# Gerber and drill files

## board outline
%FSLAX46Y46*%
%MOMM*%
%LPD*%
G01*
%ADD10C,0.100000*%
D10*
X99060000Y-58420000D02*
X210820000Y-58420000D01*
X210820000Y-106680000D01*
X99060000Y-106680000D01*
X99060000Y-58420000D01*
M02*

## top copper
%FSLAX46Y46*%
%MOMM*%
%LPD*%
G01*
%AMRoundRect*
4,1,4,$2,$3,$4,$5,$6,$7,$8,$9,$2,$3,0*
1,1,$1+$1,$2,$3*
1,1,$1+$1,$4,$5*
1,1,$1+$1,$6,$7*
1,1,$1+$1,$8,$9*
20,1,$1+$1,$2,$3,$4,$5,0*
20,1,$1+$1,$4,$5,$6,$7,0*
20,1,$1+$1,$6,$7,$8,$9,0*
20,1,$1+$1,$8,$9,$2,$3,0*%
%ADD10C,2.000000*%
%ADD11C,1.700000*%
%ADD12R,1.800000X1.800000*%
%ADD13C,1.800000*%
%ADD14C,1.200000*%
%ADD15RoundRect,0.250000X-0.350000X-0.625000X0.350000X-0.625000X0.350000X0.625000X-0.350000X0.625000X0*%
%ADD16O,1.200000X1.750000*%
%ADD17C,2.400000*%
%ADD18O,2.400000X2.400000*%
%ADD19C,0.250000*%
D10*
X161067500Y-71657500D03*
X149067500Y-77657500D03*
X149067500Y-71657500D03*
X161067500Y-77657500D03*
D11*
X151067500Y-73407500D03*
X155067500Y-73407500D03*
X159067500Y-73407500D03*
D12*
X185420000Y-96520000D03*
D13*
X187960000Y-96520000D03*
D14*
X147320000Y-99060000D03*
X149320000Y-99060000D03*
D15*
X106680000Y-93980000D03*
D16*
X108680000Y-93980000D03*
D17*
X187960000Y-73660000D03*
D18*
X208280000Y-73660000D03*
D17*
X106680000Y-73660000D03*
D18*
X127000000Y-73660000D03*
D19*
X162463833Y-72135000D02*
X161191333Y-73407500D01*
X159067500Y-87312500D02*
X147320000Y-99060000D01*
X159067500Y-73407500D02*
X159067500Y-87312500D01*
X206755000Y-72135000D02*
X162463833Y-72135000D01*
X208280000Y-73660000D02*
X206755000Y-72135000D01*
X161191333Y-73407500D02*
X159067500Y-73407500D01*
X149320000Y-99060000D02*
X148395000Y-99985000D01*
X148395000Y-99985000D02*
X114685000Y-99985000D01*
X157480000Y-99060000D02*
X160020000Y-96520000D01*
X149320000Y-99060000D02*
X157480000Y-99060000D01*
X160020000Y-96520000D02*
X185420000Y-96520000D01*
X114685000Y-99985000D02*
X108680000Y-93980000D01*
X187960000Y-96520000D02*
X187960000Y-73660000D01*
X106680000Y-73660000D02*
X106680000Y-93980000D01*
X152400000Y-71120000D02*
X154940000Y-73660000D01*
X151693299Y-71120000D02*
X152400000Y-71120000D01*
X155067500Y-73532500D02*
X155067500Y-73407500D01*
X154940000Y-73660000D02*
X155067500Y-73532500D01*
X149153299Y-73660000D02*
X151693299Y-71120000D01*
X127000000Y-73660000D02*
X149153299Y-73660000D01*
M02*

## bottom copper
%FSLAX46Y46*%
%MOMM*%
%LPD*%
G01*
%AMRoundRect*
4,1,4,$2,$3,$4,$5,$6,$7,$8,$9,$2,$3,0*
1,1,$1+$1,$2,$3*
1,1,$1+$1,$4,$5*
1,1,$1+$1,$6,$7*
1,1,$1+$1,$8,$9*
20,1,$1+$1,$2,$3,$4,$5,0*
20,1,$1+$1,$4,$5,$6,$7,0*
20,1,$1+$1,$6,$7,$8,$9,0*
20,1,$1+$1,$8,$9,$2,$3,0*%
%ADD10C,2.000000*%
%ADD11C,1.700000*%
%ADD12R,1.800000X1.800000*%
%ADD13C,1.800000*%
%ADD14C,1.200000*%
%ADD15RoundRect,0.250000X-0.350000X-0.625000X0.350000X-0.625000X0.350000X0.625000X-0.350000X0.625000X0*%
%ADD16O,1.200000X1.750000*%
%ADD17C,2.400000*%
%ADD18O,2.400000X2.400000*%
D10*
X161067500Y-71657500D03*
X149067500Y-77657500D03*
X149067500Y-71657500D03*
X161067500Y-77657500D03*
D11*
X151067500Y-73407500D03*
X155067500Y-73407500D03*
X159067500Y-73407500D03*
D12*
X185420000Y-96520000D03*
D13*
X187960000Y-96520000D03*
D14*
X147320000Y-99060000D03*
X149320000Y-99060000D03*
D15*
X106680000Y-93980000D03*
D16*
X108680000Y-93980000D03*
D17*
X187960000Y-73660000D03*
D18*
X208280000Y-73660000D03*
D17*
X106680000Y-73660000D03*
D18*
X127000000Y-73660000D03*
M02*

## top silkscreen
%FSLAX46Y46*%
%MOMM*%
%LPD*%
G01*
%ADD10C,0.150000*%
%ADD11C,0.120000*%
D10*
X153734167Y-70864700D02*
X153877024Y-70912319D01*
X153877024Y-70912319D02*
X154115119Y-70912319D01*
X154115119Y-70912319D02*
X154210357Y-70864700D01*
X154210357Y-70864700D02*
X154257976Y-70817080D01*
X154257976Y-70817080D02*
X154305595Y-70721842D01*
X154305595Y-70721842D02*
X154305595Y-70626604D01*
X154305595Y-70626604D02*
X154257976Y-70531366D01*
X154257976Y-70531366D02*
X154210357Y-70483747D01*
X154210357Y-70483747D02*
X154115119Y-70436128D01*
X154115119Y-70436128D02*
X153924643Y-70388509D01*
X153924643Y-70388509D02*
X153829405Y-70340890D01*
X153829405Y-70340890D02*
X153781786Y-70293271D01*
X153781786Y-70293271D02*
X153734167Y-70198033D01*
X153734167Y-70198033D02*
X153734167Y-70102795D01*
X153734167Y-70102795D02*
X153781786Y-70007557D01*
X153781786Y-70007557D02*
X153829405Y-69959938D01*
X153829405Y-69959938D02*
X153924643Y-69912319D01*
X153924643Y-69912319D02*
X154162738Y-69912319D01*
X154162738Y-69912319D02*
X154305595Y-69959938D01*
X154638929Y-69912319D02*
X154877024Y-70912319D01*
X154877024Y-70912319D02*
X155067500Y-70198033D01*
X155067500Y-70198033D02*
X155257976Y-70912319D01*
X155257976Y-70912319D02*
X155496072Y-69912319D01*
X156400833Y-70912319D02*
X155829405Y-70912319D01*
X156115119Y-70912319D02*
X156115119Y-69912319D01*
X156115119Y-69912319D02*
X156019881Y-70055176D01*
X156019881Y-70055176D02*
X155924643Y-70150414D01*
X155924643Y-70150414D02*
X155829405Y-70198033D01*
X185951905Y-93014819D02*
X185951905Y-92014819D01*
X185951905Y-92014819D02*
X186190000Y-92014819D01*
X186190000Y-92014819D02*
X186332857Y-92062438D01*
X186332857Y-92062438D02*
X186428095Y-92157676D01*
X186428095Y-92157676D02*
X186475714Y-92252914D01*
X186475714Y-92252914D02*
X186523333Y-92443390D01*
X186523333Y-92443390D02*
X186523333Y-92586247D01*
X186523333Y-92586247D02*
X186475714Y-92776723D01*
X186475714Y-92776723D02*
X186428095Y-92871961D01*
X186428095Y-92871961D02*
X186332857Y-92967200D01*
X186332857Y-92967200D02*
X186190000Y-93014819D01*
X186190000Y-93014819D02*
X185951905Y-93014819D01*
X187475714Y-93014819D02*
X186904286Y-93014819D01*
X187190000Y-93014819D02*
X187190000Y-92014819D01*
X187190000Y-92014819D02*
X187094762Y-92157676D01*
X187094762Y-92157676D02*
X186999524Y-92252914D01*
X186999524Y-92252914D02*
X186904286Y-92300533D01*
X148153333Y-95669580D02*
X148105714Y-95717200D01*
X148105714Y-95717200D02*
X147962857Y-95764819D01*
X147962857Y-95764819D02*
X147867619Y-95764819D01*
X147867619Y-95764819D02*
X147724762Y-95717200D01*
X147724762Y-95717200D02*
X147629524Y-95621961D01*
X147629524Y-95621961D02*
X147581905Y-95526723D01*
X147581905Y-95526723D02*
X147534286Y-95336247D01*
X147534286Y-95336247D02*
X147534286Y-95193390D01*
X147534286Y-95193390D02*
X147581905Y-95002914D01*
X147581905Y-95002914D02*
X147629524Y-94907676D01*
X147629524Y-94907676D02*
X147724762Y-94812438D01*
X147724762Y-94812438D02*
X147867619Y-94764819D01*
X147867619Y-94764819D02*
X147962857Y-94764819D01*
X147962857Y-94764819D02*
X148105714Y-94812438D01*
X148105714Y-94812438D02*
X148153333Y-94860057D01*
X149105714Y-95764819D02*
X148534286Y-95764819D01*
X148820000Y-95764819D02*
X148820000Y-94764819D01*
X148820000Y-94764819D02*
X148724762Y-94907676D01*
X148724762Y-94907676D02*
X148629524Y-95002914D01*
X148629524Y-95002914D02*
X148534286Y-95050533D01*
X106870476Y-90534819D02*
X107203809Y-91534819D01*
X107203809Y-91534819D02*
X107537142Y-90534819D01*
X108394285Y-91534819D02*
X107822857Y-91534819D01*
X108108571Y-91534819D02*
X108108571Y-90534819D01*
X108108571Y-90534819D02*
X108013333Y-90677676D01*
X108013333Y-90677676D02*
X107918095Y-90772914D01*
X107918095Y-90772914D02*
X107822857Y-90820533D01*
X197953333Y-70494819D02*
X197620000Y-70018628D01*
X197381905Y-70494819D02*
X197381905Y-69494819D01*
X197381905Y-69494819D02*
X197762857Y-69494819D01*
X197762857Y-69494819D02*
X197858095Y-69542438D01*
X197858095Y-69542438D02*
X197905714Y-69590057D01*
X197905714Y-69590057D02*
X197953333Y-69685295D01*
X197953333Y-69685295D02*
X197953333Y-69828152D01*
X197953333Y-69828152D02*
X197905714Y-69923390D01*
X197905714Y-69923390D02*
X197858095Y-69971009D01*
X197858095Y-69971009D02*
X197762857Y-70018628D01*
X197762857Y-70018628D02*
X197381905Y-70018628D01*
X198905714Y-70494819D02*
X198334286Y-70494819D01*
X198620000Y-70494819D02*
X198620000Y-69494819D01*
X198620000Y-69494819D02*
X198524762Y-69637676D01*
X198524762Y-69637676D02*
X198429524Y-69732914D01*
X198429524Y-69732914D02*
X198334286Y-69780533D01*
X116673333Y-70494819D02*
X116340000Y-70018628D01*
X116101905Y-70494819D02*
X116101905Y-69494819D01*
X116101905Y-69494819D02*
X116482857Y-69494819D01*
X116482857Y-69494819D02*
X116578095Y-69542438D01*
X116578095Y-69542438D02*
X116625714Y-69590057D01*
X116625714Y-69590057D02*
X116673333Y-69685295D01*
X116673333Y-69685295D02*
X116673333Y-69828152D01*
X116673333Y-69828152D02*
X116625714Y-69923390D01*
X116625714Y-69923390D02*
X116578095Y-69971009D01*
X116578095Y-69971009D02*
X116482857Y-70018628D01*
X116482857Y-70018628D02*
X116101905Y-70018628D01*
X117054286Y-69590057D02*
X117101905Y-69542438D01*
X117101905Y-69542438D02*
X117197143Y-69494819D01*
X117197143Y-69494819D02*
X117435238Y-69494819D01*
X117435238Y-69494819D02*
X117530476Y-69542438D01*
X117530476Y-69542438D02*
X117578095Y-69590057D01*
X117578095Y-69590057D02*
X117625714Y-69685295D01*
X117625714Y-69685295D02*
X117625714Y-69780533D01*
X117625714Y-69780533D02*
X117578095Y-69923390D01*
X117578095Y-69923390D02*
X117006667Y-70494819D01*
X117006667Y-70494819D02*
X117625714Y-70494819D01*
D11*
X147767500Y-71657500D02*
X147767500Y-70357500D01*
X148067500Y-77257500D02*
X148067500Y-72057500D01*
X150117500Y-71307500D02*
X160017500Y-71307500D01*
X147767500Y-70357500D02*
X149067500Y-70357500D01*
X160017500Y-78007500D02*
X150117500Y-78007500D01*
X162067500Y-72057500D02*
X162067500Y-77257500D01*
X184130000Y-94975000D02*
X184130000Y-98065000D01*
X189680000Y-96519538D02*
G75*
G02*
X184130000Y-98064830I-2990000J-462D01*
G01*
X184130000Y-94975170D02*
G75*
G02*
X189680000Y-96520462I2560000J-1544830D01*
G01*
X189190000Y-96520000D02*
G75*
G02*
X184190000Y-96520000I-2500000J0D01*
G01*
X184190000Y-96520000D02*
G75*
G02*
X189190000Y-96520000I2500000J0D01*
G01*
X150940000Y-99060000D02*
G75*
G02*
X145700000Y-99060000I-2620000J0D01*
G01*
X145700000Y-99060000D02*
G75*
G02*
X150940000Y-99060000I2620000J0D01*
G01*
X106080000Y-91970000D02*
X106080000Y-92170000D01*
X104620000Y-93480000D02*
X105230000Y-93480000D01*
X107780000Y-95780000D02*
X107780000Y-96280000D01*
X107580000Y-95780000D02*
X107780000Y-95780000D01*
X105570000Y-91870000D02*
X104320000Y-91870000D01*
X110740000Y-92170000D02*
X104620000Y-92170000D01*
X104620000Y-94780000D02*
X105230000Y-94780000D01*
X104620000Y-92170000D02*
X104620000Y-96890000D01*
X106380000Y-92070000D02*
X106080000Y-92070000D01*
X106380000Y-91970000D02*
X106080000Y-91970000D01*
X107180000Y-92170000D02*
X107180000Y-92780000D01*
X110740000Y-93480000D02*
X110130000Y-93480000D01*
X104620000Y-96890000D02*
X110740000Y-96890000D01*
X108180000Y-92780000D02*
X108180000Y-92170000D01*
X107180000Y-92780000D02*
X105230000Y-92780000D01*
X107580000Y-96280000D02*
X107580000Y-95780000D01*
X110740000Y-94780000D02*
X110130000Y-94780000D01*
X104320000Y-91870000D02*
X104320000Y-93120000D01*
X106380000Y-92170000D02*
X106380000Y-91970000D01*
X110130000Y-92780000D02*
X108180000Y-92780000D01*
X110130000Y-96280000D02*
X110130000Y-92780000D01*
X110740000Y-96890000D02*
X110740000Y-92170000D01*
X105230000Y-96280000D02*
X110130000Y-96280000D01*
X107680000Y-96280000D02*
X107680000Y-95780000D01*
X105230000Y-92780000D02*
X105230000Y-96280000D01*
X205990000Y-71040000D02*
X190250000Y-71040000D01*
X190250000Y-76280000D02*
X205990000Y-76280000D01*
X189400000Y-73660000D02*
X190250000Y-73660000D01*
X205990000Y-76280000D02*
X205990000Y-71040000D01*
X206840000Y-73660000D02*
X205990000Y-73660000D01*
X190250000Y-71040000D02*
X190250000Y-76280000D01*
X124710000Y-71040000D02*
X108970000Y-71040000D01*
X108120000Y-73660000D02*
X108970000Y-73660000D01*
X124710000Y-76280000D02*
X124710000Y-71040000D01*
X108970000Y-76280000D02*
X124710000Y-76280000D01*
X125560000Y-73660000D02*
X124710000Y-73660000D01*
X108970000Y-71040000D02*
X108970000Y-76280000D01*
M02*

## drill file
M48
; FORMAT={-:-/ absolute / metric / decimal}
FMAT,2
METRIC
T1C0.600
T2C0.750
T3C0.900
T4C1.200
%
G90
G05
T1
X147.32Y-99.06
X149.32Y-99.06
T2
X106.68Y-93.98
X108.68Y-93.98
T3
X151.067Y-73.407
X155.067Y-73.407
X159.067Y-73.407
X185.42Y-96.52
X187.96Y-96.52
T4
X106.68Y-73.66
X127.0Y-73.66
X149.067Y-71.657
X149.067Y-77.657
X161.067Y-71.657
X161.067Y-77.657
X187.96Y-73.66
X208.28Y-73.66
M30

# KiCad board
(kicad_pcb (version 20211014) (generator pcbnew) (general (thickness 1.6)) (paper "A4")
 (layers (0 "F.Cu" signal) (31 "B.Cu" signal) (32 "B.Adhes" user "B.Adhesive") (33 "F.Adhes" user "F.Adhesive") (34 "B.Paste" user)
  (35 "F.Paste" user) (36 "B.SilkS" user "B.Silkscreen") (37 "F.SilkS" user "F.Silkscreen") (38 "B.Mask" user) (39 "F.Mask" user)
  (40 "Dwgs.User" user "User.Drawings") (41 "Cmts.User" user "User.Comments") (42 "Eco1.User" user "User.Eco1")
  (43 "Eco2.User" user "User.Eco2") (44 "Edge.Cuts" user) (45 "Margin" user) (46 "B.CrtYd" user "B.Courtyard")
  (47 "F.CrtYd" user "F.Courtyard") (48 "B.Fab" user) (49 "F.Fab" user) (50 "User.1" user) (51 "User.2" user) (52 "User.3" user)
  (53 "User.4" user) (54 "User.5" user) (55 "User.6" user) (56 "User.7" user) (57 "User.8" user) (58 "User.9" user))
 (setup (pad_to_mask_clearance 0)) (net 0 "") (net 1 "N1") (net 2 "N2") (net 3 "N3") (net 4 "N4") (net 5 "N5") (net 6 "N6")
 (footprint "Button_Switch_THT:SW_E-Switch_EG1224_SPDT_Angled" (layer "F.Cu") (at 151.0675 73.4075)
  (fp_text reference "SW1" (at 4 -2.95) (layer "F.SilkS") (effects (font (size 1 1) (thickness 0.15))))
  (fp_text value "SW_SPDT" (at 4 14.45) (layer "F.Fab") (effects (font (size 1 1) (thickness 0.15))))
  (fp_line (start -3.3 -1.75) (end -3.3 -3.05) (layer "F.SilkS") (width 0.12))
  (fp_line (start -3 3.85) (end -3 -1.35) (layer "F.SilkS") (width 0.12))
  (fp_line (start -0.95 -2.1) (end 8.95 -2.1) (layer "F.SilkS") (width 0.12))
  (fp_line (start -3.3 -3.05) (end -2 -3.05) (layer "F.SilkS") (width 0.12))
  (fp_line (start 8.95 4.6) (end -0.95 4.6) (layer "F.SilkS") (width 0.12))
  (fp_line (start 11 -1.35) (end 11 3.85) (layer "F.SilkS") (width 0.12))
  (pad "" thru_hole circle (at 10 -1.75) (size 2 2) (drill 1.2) (layers *.Cu *.Mask))
  (pad "" thru_hole circle (at -2 4.25) (size 2 2) (drill 1.2) (layers *.Cu *.Mask))
  (pad "" thru_hole circle (at -2 -1.75) (size 2 2) (drill 1.2) (layers *.Cu *.Mask))
  (pad "" thru_hole circle (at 10 4.25) (size 2 2) (drill 1.2) (layers *.Cu *.Mask))
  (pad "1" thru_hole circle (at 0 0) (size 1.7 1.7) (drill 0.9) (layers *.Cu *.Mask) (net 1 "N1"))
  (pad "2" thru_hole circle (at 4 0) (size 1.7 1.7) (drill 0.9) (layers *.Cu *.Mask) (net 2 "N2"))
  (pad "3" thru_hole circle (at 8 0) (size 1.7 1.7) (drill 0.9) (layers *.Cu *.Mask) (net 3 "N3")))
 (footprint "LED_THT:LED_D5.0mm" (layer "F.Cu") (at 185.42 96.52)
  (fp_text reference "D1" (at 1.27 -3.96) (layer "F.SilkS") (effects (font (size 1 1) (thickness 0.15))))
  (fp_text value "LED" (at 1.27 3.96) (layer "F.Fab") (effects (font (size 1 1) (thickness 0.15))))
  (fp_line (start -1.29 -1.545) (end -1.29 1.545) (layer "F.SilkS") (width 0.12))
  (fp_arc (start 4.26 -0.000462) (mid 2.072002 2.880433) (end -1.29 1.54483) (layer "F.SilkS") (width 0.12))
  (fp_arc (start -1.29 -1.54483) (mid 2.072002 -2.880433) (end 4.26 0.000462) (layer "F.SilkS") (width 0.12))
  (fp_circle (center 1.27 0) (end 3.77 0) (layer "F.SilkS") (width 0.12) (fill none))
  (pad "1" thru_hole rect (at 0 0) (size 1.8 1.8) (drill 0.9) (layers *.Cu *.Mask) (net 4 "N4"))
  (pad "2" thru_hole circle (at 2.54 0) (size 1.8 1.8) (drill 0.9) (layers *.Cu *.Mask) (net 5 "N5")))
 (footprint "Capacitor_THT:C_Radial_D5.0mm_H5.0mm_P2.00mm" (layer "F.Cu") (at 147.32 99.06)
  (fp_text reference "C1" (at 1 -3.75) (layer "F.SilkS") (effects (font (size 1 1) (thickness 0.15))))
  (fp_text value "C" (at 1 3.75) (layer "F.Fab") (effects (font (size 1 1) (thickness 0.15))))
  (fp_circle (center 1 0) (end 3.62 0) (layer "F.SilkS") (width 0.12) (fill none))
  (pad "1" thru_hole circle (at 0 0) (size 1.2 1.2) (drill 0.6) (layers *.Cu *.Mask) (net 3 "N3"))
  (pad "2" thru_hole circle (at 2 0) (size 1.2 1.2) (drill 0.6) (layers *.Cu *.Mask) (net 4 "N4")))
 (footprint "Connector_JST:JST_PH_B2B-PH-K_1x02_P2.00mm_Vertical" (layer "F.Cu") (at 106.68 93.98)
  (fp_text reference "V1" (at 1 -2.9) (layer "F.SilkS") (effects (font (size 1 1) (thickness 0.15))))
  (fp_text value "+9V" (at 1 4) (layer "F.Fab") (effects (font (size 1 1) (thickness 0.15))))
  (fp_line (start -0.6 -2.01) (end -0.6 -1.81) (layer "F.SilkS") (width 0.12))
  (fp_line (start -2.06 -0.5) (end -1.45 -0.5) (layer "F.SilkS") (width 0.12))
  (fp_line (start 1.1 1.8) (end 1.1 2.3) (layer "F.SilkS") (width 0.12))
  (fp_line (start 0.9 1.8) (end 1.1 1.8) (layer "F.SilkS") (width 0.12))
  (fp_line (start -1.11 -2.11) (end -2.36 -2.11) (layer "F.SilkS") (width 0.12))
  (fp_line (start 4.06 -1.81) (end -2.06 -1.81) (layer "F.SilkS") (width 0.12))
  (fp_line (start -2.06 0.8) (end -1.45 0.8) (layer "F.SilkS") (width 0.12))
  (fp_line (start -2.06 -1.81) (end -2.06 2.91) (layer "F.SilkS") (width 0.12))
  (fp_line (start -0.3 -1.91) (end -0.6 -1.91) (layer "F.SilkS") (width 0.12))
  (fp_line (start -0.3 -2.01) (end -0.6 -2.01) (layer "F.SilkS") (width 0.12))
  (fp_line (start 0.5 -1.81) (end 0.5 -1.2) (layer "F.SilkS") (width 0.12))
  (fp_line (start 4.06 -0.5) (end 3.45 -0.5) (layer "F.SilkS") (width 0.12))
  (fp_line (start -2.06 2.91) (end 4.06 2.91) (layer "F.SilkS") (width 0.12))
  (fp_line (start 1.5 -1.2) (end 1.5 -1.81) (layer "F.SilkS") (width 0.12))
  (fp_line (start 0.5 -1.2) (end -1.45 -1.2) (layer "F.SilkS") (width 0.12))
  (fp_line (start 0.9 2.3) (end 0.9 1.8) (layer "F.SilkS") (width 0.12))
  (fp_line (start 4.06 0.8) (end 3.45 0.8) (layer "F.SilkS") (width 0.12))
  (fp_line (start -2.36 -2.11) (end -2.36 -0.86) (layer "F.SilkS") (width 0.12))
  (fp_line (start -0.3 -1.81) (end -0.3 -2.01) (layer "F.SilkS") (width 0.12))
  (fp_line (start 3.45 -1.2) (end 1.5 -1.2) (layer "F.SilkS") (width 0.12))
  (fp_line (start 3.45 2.3) (end 3.45 -1.2) (layer "F.SilkS") (width 0.12))
  (fp_line (start 4.06 2.91) (end 4.06 -1.81) (layer "F.SilkS") (width 0.12))
  (fp_line (start -1.45 2.3) (end 3.45 2.3) (layer "F.SilkS") (width 0.12))
  (fp_line (start 1 2.3) (end 1 1.8) (layer "F.SilkS") (width 0.12))
  (fp_line (start -1.45 -1.2) (end -1.45 2.3) (layer "F.SilkS") (width 0.12))
  (pad "1" thru_hole roundrect (at 0 0) (size 1.2 1.75) (drill 0.75) (layers *.Cu *.Mask) (roundrect_rratio 0.208333) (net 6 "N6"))
  (pad "2" thru_hole oval (at 2 0) (size 1.2 1.75) (drill 0.75) (layers *.Cu *.Mask) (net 4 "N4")))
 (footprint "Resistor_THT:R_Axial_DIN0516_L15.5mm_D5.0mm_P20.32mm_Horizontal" (layer "F.Cu") (at 187.96 73.66)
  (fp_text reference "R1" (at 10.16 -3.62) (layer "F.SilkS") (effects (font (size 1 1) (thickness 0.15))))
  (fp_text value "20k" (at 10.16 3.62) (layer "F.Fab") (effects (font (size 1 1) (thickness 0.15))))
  (fp_line (start 18.03 -2.62) (end 2.29 -2.62) (layer "F.SilkS") (width 0.12))
  (fp_line (start 2.29 2.62) (end 18.03 2.62) (layer "F.SilkS") (width 0.12))
  (fp_line (start 1.44 0) (end 2.29 0) (layer "F.SilkS") (width 0.12))
  (fp_line (start 18.03 2.62) (end 18.03 -2.62) (layer "F.SilkS") (width 0.12))
  (fp_line (start 18.88 0) (end 18.03 0) (layer "F.SilkS") (width 0.12))
  (fp_line (start 2.29 -2.62) (end 2.29 2.62) (layer "F.SilkS") (width 0.12))
  (pad "1" thru_hole circle (at 0 0) (size 2.4 2.4) (drill 1.2) (layers *.Cu *.Mask) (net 5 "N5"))
  (pad "2" thru_hole oval (at 20.32 0) (size 2.4 2.4) (drill 1.2) (layers *.Cu *.Mask) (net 3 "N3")))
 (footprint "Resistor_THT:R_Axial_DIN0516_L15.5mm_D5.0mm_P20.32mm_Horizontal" (layer "F.Cu") (at 106.68 73.66)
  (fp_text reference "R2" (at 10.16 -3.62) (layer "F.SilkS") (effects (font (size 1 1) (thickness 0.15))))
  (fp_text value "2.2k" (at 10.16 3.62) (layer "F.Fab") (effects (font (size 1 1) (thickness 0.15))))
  (fp_line (start 18.03 -2.62) (end 2.29 -2.62) (layer "F.SilkS") (width 0.12))
  (fp_line (start 1.44 0) (end 2.29 0) (layer "F.SilkS") (width 0.12))
  (fp_line (start 18.03 2.62) (end 18.03 -2.62) (layer "F.SilkS") (width 0.12))
  (fp_line (start 2.29 2.62) (end 18.03 2.62) (layer "F.SilkS") (width 0.12))
  (fp_line (start 18.88 0) (end 18.03 0) (layer "F.SilkS") (width 0.12))
  (fp_line (start 2.29 -2.62) (end 2.29 2.62) (layer "F.SilkS") (width 0.12))
  (pad "1" thru_hole circle (at 0 0) (size 2.4 2.4) (drill 1.2) (layers *.Cu *.Mask) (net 6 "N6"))
  (pad "2" thru_hole oval (at 20.32 0) (size 2.4 2.4) (drill 1.2) (layers *.Cu *.Mask) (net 2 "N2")))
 (gr_rect (start 99.06 58.42) (end 210.82 106.68) (layer "Edge.Cuts") (width 0.1) (fill none))
 (segment (start 162.463833 72.135) (end 161.191333 73.4075) (width 0.25) (layer "F.Cu") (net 3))
 (segment (start 159.0675 87.3125) (end 147.32 99.06) (width 0.25) (layer "F.Cu") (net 3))
 (segment (start 159.0675 73.4075) (end 159.0675 87.3125) (width 0.25) (layer "F.Cu") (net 3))
 (segment (start 206.755 72.135) (end 162.463833 72.135) (width 0.25) (layer "F.Cu") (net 3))
 (segment (start 208.28 73.66) (end 206.755 72.135) (width 0.25) (layer "F.Cu") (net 3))
 (segment (start 161.191333 73.4075) (end 159.0675 73.4075) (width 0.25) (layer "F.Cu") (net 3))
 (segment (start 149.32 99.06) (end 148.395 99.985) (width 0.25) (layer "F.Cu") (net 4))
 (segment (start 148.395 99.985) (end 114.685 99.985) (width 0.25) (layer "F.Cu") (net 4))
 (segment (start 157.48 99.06) (end 160.02 96.52) (width 0.25) (layer "F.Cu") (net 4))
 (segment (start 149.32 99.06) (end 157.48 99.06) (width 0.25) (layer "F.Cu") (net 4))
 (segment (start 160.02 96.52) (end 185.42 96.52) (width 0.25) (layer "F.Cu") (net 4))
 (segment (start 114.685 99.985) (end 108.68 93.98) (width 0.25) (layer "F.Cu") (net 4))
 (segment (start 187.96 96.52) (end 187.96 73.66) (width 0.25) (layer "F.Cu") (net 5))
 (segment (start 106.68 73.66) (end 106.68 93.98) (width 0.25) (layer "F.Cu") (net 6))
 (segment (start 152.4 71.12) (end 154.94 73.66) (width 0.25) (layer "F.Cu") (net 2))
 (segment (start 151.693299 71.12) (end 152.4 71.12) (width 0.25) (layer "F.Cu") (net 2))
 (segment (start 155.0675 73.5325) (end 155.0675 73.4075) (width 0.25) (layer "F.Cu") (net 2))
 (segment (start 154.94 73.66) (end 155.0675 73.5325) (width 0.25) (layer "F.Cu") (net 2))
 (segment (start 149.153299 73.66) (end 151.693299 71.12) (width 0.25) (layer "F.Cu") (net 2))
 (segment (start 127 73.66) (end 149.153299 73.66) (width 0.25) (layer "F.Cu") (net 2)))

